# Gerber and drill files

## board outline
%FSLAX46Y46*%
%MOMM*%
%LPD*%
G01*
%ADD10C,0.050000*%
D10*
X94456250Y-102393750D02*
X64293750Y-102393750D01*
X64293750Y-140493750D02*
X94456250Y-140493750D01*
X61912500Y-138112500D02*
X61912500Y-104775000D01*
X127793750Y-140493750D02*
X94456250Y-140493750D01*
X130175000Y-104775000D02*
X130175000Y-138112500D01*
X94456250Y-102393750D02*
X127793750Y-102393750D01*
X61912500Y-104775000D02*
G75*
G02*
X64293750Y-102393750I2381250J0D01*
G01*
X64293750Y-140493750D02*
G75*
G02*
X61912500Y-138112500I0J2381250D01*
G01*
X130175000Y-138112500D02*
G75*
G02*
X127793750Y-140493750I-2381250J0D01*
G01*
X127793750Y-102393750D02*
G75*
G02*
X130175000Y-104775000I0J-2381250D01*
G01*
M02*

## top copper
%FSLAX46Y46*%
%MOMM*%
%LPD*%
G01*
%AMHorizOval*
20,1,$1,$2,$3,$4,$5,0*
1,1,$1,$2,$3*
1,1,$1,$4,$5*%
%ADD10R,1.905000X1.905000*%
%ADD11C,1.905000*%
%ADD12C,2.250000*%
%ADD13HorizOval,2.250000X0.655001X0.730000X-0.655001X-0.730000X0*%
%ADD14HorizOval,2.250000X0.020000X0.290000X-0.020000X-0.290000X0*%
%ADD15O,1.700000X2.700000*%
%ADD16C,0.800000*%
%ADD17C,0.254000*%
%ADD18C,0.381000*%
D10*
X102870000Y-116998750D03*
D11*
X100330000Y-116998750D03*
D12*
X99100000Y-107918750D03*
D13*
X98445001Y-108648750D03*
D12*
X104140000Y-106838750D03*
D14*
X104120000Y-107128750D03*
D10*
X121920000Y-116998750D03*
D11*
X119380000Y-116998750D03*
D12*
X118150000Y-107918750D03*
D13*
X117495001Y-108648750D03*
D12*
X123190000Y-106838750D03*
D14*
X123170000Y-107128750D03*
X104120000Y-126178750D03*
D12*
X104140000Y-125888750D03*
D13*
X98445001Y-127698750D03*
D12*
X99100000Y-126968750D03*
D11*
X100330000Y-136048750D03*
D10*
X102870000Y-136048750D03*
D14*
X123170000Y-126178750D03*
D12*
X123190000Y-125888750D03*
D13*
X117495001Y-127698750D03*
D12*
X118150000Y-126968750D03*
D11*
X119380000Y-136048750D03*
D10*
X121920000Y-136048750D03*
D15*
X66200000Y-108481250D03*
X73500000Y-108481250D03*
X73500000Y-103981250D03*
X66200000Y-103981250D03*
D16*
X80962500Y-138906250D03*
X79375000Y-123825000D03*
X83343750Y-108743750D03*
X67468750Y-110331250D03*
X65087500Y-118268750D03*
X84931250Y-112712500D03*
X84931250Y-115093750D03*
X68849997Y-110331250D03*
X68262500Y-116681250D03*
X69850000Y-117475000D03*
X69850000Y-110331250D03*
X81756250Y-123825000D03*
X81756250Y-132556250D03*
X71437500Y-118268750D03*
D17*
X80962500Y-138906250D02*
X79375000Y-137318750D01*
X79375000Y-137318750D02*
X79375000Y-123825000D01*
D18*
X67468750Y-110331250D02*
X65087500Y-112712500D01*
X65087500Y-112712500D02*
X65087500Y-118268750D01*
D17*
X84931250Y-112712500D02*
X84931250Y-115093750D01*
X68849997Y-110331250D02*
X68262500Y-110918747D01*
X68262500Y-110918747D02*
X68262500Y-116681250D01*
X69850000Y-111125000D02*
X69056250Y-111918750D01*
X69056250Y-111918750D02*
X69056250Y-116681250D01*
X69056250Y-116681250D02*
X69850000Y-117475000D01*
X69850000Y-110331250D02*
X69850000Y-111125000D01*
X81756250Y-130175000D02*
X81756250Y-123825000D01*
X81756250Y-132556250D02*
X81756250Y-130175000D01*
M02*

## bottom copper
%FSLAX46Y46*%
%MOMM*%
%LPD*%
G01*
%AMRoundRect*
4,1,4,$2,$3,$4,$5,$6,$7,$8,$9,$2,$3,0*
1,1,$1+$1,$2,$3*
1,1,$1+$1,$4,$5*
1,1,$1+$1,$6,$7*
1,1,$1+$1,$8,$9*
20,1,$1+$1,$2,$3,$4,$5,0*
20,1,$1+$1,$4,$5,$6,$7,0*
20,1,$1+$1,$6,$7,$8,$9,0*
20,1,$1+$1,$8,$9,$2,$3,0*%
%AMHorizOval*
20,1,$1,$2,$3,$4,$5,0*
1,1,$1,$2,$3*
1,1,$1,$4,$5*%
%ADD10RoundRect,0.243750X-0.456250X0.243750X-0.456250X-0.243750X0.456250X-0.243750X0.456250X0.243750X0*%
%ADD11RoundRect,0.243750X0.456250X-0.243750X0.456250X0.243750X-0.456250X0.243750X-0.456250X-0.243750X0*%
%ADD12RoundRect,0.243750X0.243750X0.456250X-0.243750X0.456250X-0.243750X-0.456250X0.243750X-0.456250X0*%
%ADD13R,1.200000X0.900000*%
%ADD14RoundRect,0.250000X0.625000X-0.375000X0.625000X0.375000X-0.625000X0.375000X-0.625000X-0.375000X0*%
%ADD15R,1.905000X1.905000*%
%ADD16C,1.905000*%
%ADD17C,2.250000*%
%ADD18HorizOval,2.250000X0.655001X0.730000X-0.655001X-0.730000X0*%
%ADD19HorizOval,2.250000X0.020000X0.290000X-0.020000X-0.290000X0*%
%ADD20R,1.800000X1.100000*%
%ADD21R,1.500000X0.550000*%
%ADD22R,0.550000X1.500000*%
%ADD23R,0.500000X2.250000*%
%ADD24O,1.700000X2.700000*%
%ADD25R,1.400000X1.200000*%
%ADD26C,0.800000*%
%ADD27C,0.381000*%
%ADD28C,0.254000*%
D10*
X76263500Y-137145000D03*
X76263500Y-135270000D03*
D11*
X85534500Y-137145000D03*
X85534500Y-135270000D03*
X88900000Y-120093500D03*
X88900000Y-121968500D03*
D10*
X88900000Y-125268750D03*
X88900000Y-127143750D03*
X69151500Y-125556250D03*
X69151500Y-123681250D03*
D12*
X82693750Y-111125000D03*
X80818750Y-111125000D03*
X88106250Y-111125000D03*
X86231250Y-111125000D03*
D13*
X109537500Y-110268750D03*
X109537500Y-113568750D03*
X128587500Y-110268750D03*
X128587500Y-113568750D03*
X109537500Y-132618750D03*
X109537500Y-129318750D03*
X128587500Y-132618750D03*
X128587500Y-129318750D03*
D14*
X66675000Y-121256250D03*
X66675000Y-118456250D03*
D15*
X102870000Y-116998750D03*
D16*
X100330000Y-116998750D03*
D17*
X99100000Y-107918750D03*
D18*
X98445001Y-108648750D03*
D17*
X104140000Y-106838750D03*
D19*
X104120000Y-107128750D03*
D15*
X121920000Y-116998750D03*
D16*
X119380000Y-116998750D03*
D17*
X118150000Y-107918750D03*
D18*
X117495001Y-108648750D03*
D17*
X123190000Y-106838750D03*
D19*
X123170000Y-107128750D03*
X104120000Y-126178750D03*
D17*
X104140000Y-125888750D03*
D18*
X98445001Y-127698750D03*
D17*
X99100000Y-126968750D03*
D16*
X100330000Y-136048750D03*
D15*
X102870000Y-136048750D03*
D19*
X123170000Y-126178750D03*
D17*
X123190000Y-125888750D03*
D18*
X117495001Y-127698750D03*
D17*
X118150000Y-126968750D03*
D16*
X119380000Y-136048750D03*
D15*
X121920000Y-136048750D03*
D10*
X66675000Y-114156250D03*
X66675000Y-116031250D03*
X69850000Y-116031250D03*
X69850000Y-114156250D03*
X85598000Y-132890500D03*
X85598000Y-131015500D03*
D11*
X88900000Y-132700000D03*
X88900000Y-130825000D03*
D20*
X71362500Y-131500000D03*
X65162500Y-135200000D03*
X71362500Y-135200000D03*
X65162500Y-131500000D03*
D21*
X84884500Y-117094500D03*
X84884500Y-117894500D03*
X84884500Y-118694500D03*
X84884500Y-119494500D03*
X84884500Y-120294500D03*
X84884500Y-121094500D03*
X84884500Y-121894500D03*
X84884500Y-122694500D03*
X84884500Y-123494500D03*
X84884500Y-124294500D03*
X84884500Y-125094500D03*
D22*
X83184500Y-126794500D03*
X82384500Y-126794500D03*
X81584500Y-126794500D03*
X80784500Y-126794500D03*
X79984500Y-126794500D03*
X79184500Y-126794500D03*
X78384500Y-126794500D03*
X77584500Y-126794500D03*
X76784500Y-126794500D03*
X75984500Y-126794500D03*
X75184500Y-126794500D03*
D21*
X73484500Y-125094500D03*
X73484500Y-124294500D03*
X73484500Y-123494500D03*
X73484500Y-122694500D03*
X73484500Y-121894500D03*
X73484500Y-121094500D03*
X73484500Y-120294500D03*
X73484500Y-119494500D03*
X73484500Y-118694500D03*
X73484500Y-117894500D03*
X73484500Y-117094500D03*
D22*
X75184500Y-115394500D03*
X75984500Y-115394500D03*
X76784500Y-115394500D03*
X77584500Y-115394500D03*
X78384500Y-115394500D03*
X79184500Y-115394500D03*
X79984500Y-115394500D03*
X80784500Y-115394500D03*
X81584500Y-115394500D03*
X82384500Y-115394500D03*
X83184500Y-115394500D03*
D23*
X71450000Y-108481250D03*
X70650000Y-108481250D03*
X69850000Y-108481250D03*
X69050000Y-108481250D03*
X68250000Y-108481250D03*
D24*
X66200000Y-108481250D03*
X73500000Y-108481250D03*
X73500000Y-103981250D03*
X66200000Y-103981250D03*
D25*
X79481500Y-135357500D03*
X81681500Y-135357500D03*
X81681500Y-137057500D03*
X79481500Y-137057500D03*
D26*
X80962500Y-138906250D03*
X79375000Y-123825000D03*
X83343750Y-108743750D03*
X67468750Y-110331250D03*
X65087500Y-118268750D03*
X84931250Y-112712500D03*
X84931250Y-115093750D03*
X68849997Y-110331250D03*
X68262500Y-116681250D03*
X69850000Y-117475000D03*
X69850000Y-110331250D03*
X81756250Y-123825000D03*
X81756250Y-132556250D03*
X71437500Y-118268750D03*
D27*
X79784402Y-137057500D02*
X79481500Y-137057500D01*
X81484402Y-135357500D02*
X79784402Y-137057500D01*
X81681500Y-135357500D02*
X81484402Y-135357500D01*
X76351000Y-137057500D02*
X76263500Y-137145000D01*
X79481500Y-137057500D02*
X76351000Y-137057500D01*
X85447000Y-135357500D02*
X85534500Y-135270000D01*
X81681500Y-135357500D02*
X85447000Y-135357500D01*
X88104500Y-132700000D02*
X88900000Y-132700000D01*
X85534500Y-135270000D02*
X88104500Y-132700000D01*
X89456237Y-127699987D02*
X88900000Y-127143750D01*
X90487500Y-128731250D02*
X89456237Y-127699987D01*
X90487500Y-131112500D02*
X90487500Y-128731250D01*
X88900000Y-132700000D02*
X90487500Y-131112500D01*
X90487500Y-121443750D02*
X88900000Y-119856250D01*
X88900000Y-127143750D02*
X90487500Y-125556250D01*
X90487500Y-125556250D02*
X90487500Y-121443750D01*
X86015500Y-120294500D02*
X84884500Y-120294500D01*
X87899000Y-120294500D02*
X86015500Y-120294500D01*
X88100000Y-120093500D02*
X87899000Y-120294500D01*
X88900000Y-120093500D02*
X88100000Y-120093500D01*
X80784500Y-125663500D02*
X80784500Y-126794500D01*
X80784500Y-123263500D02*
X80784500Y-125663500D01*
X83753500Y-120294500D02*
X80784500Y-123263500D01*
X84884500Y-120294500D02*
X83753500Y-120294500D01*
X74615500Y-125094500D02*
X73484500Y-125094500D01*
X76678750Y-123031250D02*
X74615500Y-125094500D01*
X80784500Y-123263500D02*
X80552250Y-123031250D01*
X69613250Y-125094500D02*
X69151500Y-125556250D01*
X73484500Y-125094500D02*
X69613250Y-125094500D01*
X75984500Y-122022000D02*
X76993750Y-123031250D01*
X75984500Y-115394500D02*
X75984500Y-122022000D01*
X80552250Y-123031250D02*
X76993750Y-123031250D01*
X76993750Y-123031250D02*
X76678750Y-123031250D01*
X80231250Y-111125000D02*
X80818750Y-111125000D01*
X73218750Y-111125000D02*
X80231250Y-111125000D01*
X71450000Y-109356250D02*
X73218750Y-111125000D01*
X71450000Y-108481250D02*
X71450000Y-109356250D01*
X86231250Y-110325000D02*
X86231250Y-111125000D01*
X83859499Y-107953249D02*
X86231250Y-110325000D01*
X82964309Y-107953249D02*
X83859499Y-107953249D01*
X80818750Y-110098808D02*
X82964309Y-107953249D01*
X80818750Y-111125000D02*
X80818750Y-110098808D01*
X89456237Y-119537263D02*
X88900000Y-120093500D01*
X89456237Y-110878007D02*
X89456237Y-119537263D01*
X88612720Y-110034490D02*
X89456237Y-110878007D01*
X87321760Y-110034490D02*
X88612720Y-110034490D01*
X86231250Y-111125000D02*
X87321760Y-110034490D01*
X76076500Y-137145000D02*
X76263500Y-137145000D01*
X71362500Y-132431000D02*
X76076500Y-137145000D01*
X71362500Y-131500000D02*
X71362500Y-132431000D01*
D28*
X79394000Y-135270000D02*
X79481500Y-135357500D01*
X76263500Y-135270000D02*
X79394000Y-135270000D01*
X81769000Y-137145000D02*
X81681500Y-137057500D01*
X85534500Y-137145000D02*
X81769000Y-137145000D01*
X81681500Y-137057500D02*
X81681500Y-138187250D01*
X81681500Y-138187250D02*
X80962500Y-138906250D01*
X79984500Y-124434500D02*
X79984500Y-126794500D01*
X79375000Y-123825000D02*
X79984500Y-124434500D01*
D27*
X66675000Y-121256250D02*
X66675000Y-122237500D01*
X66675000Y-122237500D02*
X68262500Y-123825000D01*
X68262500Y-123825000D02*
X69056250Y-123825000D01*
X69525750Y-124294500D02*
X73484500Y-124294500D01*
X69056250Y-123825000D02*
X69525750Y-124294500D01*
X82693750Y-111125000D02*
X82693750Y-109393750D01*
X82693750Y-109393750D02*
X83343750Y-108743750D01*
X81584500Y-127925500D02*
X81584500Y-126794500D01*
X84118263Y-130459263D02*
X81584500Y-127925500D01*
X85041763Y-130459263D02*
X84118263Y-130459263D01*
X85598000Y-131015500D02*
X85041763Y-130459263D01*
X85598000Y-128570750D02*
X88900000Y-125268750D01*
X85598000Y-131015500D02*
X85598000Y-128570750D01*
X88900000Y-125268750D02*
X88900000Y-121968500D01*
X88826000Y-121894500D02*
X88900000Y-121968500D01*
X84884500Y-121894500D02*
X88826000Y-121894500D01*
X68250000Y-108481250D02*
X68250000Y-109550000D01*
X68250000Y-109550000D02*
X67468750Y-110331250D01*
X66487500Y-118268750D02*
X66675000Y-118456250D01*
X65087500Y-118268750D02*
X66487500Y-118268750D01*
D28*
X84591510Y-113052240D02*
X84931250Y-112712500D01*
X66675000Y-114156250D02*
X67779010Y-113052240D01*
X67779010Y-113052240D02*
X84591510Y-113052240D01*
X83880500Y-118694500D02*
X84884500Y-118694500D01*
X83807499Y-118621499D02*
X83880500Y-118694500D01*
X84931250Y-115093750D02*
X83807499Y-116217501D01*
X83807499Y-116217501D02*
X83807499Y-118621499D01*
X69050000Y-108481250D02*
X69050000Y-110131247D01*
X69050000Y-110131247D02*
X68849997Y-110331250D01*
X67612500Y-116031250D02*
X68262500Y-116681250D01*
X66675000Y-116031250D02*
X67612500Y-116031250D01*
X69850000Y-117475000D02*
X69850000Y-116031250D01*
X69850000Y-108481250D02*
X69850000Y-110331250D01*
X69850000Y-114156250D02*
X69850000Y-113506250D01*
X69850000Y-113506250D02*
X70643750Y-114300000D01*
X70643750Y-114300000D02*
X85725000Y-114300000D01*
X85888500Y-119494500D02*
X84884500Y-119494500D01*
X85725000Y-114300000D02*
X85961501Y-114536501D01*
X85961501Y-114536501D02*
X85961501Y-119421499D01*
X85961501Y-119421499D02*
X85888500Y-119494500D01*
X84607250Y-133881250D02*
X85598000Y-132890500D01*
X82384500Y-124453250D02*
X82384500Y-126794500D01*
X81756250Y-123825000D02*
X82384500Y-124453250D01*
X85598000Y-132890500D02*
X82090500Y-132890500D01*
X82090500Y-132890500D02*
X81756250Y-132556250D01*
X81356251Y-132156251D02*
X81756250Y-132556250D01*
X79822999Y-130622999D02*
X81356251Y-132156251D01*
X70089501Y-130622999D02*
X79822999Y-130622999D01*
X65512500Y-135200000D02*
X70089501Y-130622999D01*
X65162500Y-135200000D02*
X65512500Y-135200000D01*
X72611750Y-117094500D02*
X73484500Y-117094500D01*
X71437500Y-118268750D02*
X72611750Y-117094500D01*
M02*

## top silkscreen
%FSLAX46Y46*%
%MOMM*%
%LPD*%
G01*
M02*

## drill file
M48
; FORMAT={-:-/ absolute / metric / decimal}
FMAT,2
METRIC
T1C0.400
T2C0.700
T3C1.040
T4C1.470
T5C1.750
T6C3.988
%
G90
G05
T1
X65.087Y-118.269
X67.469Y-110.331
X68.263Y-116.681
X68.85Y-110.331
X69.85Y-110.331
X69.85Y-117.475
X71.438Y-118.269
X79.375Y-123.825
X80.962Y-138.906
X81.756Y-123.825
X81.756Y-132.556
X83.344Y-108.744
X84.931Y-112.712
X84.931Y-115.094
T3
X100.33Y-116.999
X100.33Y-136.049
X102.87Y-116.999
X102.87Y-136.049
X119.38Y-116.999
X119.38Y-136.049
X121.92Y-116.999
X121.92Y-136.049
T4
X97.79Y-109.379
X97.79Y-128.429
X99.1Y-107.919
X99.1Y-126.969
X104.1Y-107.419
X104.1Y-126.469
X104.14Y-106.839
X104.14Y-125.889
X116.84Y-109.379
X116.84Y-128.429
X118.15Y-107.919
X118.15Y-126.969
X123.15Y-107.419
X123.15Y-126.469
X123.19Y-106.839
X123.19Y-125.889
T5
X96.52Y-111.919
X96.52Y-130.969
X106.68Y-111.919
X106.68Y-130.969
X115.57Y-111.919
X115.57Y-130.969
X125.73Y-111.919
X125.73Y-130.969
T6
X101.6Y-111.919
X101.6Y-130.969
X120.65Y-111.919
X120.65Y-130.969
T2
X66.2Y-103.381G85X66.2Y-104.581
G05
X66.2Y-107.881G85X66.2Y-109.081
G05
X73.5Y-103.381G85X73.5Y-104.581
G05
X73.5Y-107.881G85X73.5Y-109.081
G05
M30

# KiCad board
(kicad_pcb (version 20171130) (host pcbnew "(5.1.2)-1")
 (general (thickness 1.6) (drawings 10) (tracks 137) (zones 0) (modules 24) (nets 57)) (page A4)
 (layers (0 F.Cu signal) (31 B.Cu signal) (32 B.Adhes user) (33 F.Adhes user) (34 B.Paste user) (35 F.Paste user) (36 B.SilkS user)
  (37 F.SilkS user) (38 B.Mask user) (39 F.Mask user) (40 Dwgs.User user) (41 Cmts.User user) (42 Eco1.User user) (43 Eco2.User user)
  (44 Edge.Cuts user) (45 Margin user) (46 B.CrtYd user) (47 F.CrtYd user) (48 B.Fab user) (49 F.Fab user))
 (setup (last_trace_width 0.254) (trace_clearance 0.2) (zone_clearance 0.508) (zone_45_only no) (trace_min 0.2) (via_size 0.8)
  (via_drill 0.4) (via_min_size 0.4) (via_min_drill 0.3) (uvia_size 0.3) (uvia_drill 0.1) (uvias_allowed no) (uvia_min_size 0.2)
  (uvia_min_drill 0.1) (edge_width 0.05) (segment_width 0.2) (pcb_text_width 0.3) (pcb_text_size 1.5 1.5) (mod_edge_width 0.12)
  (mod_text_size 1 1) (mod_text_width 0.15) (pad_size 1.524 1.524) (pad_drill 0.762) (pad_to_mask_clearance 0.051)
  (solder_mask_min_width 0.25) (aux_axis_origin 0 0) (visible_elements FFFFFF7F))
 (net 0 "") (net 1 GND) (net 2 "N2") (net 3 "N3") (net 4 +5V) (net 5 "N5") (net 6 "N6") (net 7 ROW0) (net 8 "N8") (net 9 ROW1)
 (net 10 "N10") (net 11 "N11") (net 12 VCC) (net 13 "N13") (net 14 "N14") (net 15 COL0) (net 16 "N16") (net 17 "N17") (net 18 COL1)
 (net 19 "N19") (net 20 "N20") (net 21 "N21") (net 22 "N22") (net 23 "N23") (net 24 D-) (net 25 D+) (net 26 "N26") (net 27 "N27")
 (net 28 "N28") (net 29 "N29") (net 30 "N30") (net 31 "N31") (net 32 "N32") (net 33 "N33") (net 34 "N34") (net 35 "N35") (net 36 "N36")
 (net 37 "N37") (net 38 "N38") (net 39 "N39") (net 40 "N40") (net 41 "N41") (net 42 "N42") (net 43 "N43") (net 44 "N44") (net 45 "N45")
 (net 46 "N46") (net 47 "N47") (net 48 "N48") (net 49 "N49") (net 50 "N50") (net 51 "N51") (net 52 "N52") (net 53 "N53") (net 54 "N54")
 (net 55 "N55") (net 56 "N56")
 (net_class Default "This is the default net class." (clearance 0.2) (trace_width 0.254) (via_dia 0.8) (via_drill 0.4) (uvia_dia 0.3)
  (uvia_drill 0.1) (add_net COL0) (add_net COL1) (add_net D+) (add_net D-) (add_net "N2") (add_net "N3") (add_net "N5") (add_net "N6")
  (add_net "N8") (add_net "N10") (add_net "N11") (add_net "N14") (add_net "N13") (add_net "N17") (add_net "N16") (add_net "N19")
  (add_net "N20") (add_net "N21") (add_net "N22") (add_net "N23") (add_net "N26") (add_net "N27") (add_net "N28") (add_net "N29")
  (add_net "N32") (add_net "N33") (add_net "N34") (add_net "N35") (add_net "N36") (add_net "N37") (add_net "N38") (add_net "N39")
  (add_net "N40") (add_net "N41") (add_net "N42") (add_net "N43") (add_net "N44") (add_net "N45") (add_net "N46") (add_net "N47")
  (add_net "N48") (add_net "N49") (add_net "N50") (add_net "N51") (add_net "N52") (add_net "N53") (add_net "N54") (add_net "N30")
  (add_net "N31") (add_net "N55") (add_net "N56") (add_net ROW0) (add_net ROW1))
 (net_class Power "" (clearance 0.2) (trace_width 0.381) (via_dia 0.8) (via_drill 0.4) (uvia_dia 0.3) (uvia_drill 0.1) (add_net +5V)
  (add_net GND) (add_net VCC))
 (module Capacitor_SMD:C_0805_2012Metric (layer B.Cu) (at 76.2635 136.2075 270)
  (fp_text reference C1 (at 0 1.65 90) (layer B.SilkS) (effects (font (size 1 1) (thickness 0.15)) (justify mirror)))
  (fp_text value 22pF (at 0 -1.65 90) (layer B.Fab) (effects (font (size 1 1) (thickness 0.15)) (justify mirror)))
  (pad 2 smd roundrect (at 0.9375 0 270) (size 0.975 1.4) (layers B.Cu B.Paste B.Mask) (roundrect_rratio 0.25) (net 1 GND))
  (pad 1 smd roundrect (at -0.9375 0 270) (size 0.975 1.4) (layers B.Cu B.Paste B.Mask) (roundrect_rratio 0.25) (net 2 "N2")))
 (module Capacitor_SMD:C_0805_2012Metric (layer B.Cu) (at 85.5345 136.2075 90)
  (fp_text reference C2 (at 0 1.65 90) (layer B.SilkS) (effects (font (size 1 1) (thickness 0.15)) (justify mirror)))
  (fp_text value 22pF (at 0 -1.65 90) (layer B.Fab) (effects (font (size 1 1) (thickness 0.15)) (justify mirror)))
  (pad 1 smd roundrect (at -0.9375 0 90) (size 0.975 1.4) (layers B.Cu B.Paste B.Mask) (roundrect_rratio 0.25) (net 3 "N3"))
  (pad 2 smd roundrect (at 0.9375 0 90) (size 0.975 1.4) (layers B.Cu B.Paste B.Mask) (roundrect_rratio 0.25) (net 1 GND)))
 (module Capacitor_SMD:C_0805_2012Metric (layer B.Cu) (at 88.9 121.031 90)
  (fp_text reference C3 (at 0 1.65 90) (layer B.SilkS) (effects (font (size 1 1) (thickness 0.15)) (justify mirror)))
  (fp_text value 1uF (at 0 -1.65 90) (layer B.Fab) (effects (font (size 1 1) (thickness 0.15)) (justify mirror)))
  (pad 2 smd roundrect (at 0.9375 0 90) (size 0.975 1.4) (layers B.Cu B.Paste B.Mask) (roundrect_rratio 0.25) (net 1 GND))
  (pad 1 smd roundrect (at -0.9375 0 90) (size 0.975 1.4) (layers B.Cu B.Paste B.Mask) (roundrect_rratio 0.25) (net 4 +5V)))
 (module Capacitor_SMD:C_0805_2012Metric (layer B.Cu) (at 88.9 126.20625 270)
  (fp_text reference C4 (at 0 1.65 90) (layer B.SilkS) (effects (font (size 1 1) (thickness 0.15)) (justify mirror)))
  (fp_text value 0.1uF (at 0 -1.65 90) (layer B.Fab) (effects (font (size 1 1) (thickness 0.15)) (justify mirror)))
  (pad 1 smd roundrect (at -0.9375 0 270) (size 0.975 1.4) (layers B.Cu B.Paste B.Mask) (roundrect_rratio 0.25) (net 4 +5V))
  (pad 2 smd roundrect (at 0.9375 0 270) (size 0.975 1.4) (layers B.Cu B.Paste B.Mask) (roundrect_rratio 0.25) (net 1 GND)))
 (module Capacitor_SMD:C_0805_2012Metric (layer B.Cu) (at 69.1515 124.61875 270)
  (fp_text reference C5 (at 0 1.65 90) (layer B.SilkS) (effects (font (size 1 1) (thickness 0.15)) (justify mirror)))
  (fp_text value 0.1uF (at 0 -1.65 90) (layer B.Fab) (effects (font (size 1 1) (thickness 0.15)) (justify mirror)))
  (pad 2 smd roundrect (at 0.9375 0 270) (size 0.975 1.4) (layers B.Cu B.Paste B.Mask) (roundrect_rratio 0.25) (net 1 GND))
  (pad 1 smd roundrect (at -0.9375 0 270) (size 0.975 1.4) (layers B.Cu B.Paste B.Mask) (roundrect_rratio 0.25) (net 4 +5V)))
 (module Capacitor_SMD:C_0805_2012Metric (layer B.Cu) (at 81.75625 111.125 180)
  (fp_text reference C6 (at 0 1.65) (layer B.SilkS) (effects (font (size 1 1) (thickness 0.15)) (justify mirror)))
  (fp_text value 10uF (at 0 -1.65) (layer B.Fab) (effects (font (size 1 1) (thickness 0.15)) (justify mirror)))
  (pad 1 smd roundrect (at -0.9375 0 180) (size 0.975 1.4) (layers B.Cu B.Paste B.Mask) (roundrect_rratio 0.25) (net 4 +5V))
  (pad 2 smd roundrect (at 0.9375 0 180) (size 0.975 1.4) (layers B.Cu B.Paste B.Mask) (roundrect_rratio 0.25) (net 1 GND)))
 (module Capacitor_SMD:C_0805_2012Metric (layer B.Cu) (at 87.16875 111.125 180)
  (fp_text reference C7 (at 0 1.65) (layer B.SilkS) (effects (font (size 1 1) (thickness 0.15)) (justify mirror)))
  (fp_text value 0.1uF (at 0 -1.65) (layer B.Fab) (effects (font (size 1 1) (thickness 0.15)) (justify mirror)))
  (pad 1 smd roundrect (at -0.9375 0 180) (size 0.975 1.4) (layers B.Cu B.Paste B.Mask) (roundrect_rratio 0.25) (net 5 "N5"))
  (pad 2 smd roundrect (at 0.9375 0 180) (size 0.975 1.4) (layers B.Cu B.Paste B.Mask) (roundrect_rratio 0.25) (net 1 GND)))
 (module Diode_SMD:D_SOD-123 (layer B.Cu) (at 109.5375 111.91875 90)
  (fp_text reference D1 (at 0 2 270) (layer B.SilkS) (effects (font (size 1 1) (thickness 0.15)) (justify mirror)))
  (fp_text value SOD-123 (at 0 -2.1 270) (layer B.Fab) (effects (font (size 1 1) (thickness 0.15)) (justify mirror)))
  (pad 2 smd rect (at 1.65 0 90) (size 0.9 1.2) (layers B.Cu B.Paste B.Mask) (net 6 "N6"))
  (pad 1 smd rect (at -1.65 0 90) (size 0.9 1.2) (layers B.Cu B.Paste B.Mask) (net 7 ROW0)))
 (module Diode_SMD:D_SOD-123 (layer B.Cu) (at 128.5875 111.91875 90)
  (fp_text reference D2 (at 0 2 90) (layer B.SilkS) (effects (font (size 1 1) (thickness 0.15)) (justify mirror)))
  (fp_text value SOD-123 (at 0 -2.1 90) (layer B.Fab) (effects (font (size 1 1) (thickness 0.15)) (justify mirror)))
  (pad 2 smd rect (at 1.65 0 90) (size 0.9 1.2) (layers B.Cu B.Paste B.Mask) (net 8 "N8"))
  (pad 1 smd rect (at -1.65 0 90) (size 0.9 1.2) (layers B.Cu B.Paste B.Mask) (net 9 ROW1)))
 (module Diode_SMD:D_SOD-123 (layer B.Cu) (at 109.5375 130.96875 90)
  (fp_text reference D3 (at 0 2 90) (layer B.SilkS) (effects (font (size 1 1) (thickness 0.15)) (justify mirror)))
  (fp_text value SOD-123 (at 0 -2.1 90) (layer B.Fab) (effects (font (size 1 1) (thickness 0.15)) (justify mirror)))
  (pad 1 smd rect (at -1.65 0 90) (size 0.9 1.2) (layers B.Cu B.Paste B.Mask) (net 7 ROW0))
  (pad 2 smd rect (at 1.65 0 90) (size 0.9 1.2) (layers B.Cu B.Paste B.Mask) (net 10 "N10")))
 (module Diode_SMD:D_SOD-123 (layer B.Cu) (at 128.5875 130.96875 90)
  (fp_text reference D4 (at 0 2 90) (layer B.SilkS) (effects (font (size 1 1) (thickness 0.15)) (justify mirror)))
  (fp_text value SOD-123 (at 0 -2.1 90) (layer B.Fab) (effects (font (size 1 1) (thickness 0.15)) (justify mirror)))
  (pad 1 smd rect (at -1.65 0 90) (size 0.9 1.2) (layers B.Cu B.Paste B.Mask) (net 9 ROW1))
  (pad 2 smd rect (at 1.65 0 90) (size 0.9 1.2) (layers B.Cu B.Paste B.Mask) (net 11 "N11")))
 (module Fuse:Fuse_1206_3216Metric (layer B.Cu) (at 66.675 119.85625 90)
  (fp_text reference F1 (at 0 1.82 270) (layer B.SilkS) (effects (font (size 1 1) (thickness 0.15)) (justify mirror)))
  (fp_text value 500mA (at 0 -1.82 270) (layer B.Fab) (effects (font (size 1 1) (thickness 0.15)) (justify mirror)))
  (pad 1 smd roundrect (at -1.4 0 90) (size 1.25 1.75) (layers B.Cu B.Paste B.Mask) (roundrect_rratio 0.2) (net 4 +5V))
  (pad 2 smd roundrect (at 1.4 0 90) (size 1.25 1.75) (layers B.Cu B.Paste B.Mask) (roundrect_rratio 0.2) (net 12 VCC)))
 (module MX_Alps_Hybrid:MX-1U (layer F.Cu) (at 101.6 111.91875)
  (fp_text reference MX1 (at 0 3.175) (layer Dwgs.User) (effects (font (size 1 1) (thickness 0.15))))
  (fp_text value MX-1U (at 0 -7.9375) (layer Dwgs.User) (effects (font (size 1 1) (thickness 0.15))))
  (pad "" np_thru_hole circle (at 5.08 0 48.0996) (size 1.75 1.75) (drill 1.75) (layers *.Cu *.Mask))
  (pad "" np_thru_hole circle (at -5.08 0 48.0996) (size 1.75 1.75) (drill 1.75) (layers *.Cu *.Mask))
  (pad 4 thru_hole rect (at 1.27 5.08) (size 1.905 1.905) (drill 1.04) (layers *.Cu B.Mask) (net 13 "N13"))
  (pad 3 thru_hole circle (at -1.27 5.08) (size 1.905 1.905) (drill 1.04) (layers *.Cu B.Mask) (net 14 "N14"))
  (pad 1 thru_hole circle (at -2.5 -4) (size 2.25 2.25) (drill 1.47) (layers *.Cu B.Mask) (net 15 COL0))
  (pad "" np_thru_hole circle (at 0 0) (size 3.9878 3.9878) (drill 3.9878) (layers *.Cu *.Mask))
  (pad 1 thru_hole oval (at -3.81 -2.54 48.0996) (size 4.211556 2.25) (drill 1.47 (offset 0.980778 0)) (layers *.Cu B.Mask) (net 15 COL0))
  (pad 2 thru_hole circle (at 2.54 -5.08) (size 2.25 2.25) (drill 1.47) (layers *.Cu B.Mask) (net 6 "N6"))
  (pad 2 thru_hole oval (at 2.5 -4.5 86.0548) (size 2.831378 2.25) (drill 1.47 (offset 0.290689 0)) (layers *.Cu B.Mask) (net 6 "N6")))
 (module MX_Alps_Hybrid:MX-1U (layer F.Cu) (at 120.65 111.91875)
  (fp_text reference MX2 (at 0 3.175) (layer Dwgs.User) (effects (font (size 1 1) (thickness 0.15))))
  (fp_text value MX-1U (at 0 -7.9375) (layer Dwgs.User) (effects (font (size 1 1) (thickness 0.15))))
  (pad "" np_thru_hole circle (at 5.08 0 48.0996) (size 1.75 1.75) (drill 1.75) (layers *.Cu *.Mask))
  (pad "" np_thru_hole circle (at -5.08 0 48.0996) (size 1.75 1.75) (drill 1.75) (layers *.Cu *.Mask))
  (pad 4 thru_hole rect (at 1.27 5.08) (size 1.905 1.905) (drill 1.04) (layers *.Cu B.Mask) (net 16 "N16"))
  (pad 3 thru_hole circle (at -1.27 5.08) (size 1.905 1.905) (drill 1.04) (layers *.Cu B.Mask) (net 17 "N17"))
  (pad 1 thru_hole circle (at -2.5 -4) (size 2.25 2.25) (drill 1.47) (layers *.Cu B.Mask) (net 15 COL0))
  (pad "" np_thru_hole circle (at 0 0) (size 3.9878 3.9878) (drill 3.9878) (layers *.Cu *.Mask))
  (pad 1 thru_hole oval (at -3.81 -2.54 48.0996) (size 4.211556 2.25) (drill 1.47 (offset 0.980778 0)) (layers *.Cu B.Mask) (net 15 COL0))
  (pad 2 thru_hole circle (at 2.54 -5.08) (size 2.25 2.25) (drill 1.47) (layers *.Cu B.Mask) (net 8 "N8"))
  (pad 2 thru_hole oval (at 2.5 -4.5 86.0548) (size 2.831378 2.25) (drill 1.47 (offset 0.290689 0)) (layers *.Cu B.Mask) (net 8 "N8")))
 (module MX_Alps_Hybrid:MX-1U (layer F.Cu) (at 101.6 130.96875)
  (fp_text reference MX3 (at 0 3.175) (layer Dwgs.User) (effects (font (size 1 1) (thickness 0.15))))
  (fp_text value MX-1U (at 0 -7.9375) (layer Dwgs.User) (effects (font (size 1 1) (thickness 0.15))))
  (pad 2 thru_hole oval (at 2.5 -4.5 86.0548) (size 2.831378 2.25) (drill 1.47 (offset 0.290689 0)) (layers *.Cu B.Mask) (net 10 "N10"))
  (pad 2 thru_hole circle (at 2.54 -5.08) (size 2.25 2.25) (drill 1.47) (layers *.Cu B.Mask) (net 10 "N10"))
  (pad 1 thru_hole oval (at -3.81 -2.54 48.0996) (size 4.211556 2.25) (drill 1.47 (offset 0.980778 0)) (layers *.Cu B.Mask) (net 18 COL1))
  (pad "" np_thru_hole circle (at 0 0) (size 3.9878 3.9878) (drill 3.9878) (layers *.Cu *.Mask))
  (pad 1 thru_hole circle (at -2.5 -4) (size 2.25 2.25) (drill 1.47) (layers *.Cu B.Mask) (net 18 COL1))
  (pad 3 thru_hole circle (at -1.27 5.08) (size 1.905 1.905) (drill 1.04) (layers *.Cu B.Mask) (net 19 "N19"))
  (pad 4 thru_hole rect (at 1.27 5.08) (size 1.905 1.905) (drill 1.04) (layers *.Cu B.Mask) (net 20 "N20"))
  (pad "" np_thru_hole circle (at -5.08 0 48.0996) (size 1.75 1.75) (drill 1.75) (layers *.Cu *.Mask))
  (pad "" np_thru_hole circle (at 5.08 0 48.0996) (size 1.75 1.75) (drill 1.75) (layers *.Cu *.Mask)))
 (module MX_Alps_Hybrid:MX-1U (layer F.Cu) (at 120.65 130.96875)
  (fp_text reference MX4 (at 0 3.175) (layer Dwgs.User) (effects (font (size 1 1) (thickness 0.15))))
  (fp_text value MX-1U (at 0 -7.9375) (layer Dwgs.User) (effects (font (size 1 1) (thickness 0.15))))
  (pad 2 thru_hole oval (at 2.5 -4.5 86.0548) (size 2.831378 2.25) (drill 1.47 (offset 0.290689 0)) (layers *.Cu B.Mask) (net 11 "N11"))
  (pad 2 thru_hole circle (at 2.54 -5.08) (size 2.25 2.25) (drill 1.47) (layers *.Cu B.Mask) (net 11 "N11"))
  (pad 1 thru_hole oval (at -3.81 -2.54 48.0996) (size 4.211556 2.25) (drill 1.47 (offset 0.980778 0)) (layers *.Cu B.Mask) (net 18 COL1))
  (pad "" np_thru_hole circle (at 0 0) (size 3.9878 3.9878) (drill 3.9878) (layers *.Cu *.Mask))
  (pad 1 thru_hole circle (at -2.5 -4) (size 2.25 2.25) (drill 1.47) (layers *.Cu B.Mask) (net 18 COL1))
  (pad 3 thru_hole circle (at -1.27 5.08) (size 1.905 1.905) (drill 1.04) (layers *.Cu B.Mask) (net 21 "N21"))
  (pad 4 thru_hole rect (at 1.27 5.08) (size 1.905 1.905) (drill 1.04) (layers *.Cu B.Mask) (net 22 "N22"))
  (pad "" np_thru_hole circle (at -5.08 0 48.0996) (size 1.75 1.75) (drill 1.75) (layers *.Cu *.Mask))
  (pad "" np_thru_hole circle (at 5.08 0 48.0996) (size 1.75 1.75) (drill 1.75) (layers *.Cu *.Mask)))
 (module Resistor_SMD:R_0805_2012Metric (layer B.Cu) (at 66.675 115.09375 270)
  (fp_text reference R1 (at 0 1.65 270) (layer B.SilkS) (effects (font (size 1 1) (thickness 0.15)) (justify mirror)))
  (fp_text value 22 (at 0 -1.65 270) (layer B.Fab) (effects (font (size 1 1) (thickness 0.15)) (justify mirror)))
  (pad 1 smd roundrect (at -0.9375 0 270) (size 0.975 1.4) (layers B.Cu B.Paste B.Mask) (roundrect_rratio 0.25) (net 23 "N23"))
  (pad 2 smd roundrect (at 0.9375 0 270) (size 0.975 1.4) (layers B.Cu B.Paste B.Mask) (roundrect_rratio 0.25) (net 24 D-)))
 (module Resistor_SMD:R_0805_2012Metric (layer B.Cu) (at 69.85 115.09375 270)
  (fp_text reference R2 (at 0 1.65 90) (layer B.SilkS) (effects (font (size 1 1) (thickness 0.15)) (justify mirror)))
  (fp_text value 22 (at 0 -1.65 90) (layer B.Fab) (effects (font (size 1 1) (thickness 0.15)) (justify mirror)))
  (pad 2 smd roundrect (at 0.9375 0 270) (size 0.975 1.4) (layers B.Cu B.Paste B.Mask) (roundrect_rratio 0.25) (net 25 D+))
  (pad 1 smd roundrect (at -0.9375 0 270) (size 0.975 1.4) (layers B.Cu B.Paste B.Mask) (roundrect_rratio 0.25) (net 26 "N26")))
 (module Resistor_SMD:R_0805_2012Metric (layer B.Cu) (at 85.598 131.953 270)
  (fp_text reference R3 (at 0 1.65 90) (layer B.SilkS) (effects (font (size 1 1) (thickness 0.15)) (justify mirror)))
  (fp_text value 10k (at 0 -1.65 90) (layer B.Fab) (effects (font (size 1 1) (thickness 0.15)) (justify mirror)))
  (pad 2 smd roundrect (at 0.9375 0 270) (size 0.975 1.4) (layers B.Cu B.Paste B.Mask) (roundrect_rratio 0.25) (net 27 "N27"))
  (pad 1 smd roundrect (at -0.9375 0 270) (size 0.975 1.4) (layers B.Cu B.Paste B.Mask) (roundrect_rratio 0.25) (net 4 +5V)))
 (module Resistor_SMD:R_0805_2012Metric (layer B.Cu) (at 88.9 131.7625 90)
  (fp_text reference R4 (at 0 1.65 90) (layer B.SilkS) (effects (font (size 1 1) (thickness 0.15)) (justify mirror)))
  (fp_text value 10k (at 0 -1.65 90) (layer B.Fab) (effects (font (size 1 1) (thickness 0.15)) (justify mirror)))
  (pad 1 smd roundrect (at -0.9375 0 90) (size 0.975 1.4) (layers B.Cu B.Paste B.Mask) (roundrect_rratio 0.25) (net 1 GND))
  (pad 2 smd roundrect (at 0.9375 0 90) (size 0.975 1.4) (layers B.Cu B.Paste B.Mask) (roundrect_rratio 0.25) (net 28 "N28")))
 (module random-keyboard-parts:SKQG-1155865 (layer B.Cu) (at 68.2625 133.35)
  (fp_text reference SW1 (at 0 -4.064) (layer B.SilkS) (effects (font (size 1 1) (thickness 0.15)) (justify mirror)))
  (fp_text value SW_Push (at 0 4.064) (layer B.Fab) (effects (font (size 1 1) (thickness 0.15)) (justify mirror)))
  (pad 1 smd rect (at 3.1 -1.85) (size 1.8 1.1) (layers B.Cu B.Paste B.Mask) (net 1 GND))
  (pad 2 smd rect (at -3.1 1.85) (size 1.8 1.1) (layers B.Cu B.Paste B.Mask) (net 27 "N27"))
  (pad 3 smd rect (at 3.1 1.85) (size 1.8 1.1) (layers B.Cu B.Paste B.Mask))
  (pad 4 smd rect (at -3.1 -1.85) (size 1.8 1.1) (layers B.Cu B.Paste B.Mask)))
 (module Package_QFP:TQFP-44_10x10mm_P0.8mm (layer B.Cu) (at 79.1845 121.0945 180)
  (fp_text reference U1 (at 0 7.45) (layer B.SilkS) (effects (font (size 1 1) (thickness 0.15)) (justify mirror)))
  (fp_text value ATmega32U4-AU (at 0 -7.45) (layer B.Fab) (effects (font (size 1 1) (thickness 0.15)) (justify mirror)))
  (pad 1 smd rect (at -5.7 4 180) (size 1.5 0.55) (layers B.Cu B.Paste B.Mask) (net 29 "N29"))
  (pad 2 smd rect (at -5.7 3.2 180) (size 1.5 0.55) (layers B.Cu B.Paste B.Mask) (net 4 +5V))
  (pad 3 smd rect (at -5.7 2.4 180) (size 1.5 0.55) (layers B.Cu B.Paste B.Mask) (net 23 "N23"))
  (pad 4 smd rect (at -5.7 1.6 180) (size 1.5 0.55) (layers B.Cu B.Paste B.Mask) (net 26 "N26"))
  (pad 5 smd rect (at -5.7 0.8 180) (size 1.5 0.55) (layers B.Cu B.Paste B.Mask) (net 1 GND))
  (pad 6 smd rect (at -5.7 0 180) (size 1.5 0.55) (layers B.Cu B.Paste B.Mask) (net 5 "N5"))
  (pad 7 smd rect (at -5.7 -0.8 180) (size 1.5 0.55) (layers B.Cu B.Paste B.Mask) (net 4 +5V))
  (pad 8 smd rect (at -5.7 -1.6 180) (size 1.5 0.55) (layers B.Cu B.Paste B.Mask) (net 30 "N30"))
  (pad 9 smd rect (at -5.7 -2.4 180) (size 1.5 0.55) (layers B.Cu B.Paste B.Mask) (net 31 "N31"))
  (pad 10 smd rect (at -5.7 -3.2 180) (size 1.5 0.55) (layers B.Cu B.Paste B.Mask) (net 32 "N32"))
  (pad 11 smd rect (at -5.7 -4 180) (size 1.5 0.55) (layers B.Cu B.Paste B.Mask) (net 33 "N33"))
  (pad 12 smd rect (at -4 -5.7 90) (size 1.5 0.55) (layers B.Cu B.Paste B.Mask) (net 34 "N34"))
  (pad 13 smd rect (at -3.2 -5.7 90) (size 1.5 0.55) (layers B.Cu B.Paste B.Mask) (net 27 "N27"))
  (pad 14 smd rect (at -2.4 -5.7 90) (size 1.5 0.55) (layers B.Cu B.Paste B.Mask) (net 4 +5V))
  (pad 15 smd rect (at -1.6 -5.7 90) (size 1.5 0.55) (layers B.Cu B.Paste B.Mask) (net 1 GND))
  (pad 16 smd rect (at -0.8 -5.7 90) (size 1.5 0.55) (layers B.Cu B.Paste B.Mask) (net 3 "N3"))
  (pad 17 smd rect (at 0 -5.7 90) (size 1.5 0.55) (layers B.Cu B.Paste B.Mask) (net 2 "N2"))
  (pad 18 smd rect (at 0.8 -5.7 90) (size 1.5 0.55) (layers B.Cu B.Paste B.Mask) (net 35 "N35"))
  (pad 19 smd rect (at 1.6 -5.7 90) (size 1.5 0.55) (layers B.Cu B.Paste B.Mask) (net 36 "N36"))
  (pad 20 smd rect (at 2.4 -5.7 90) (size 1.5 0.55) (layers B.Cu B.Paste B.Mask) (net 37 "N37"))
  (pad 21 smd rect (at 3.2 -5.7 90) (size 1.5 0.55) (layers B.Cu B.Paste B.Mask) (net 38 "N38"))
  (pad 22 smd rect (at 4 -5.7 90) (size 1.5 0.55) (layers B.Cu B.Paste B.Mask) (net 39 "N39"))
  (pad 23 smd rect (at 5.7 -4 180) (size 1.5 0.55) (layers B.Cu B.Paste B.Mask) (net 1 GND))
  (pad 24 smd rect (at 5.7 -3.2 180) (size 1.5 0.55) (layers B.Cu B.Paste B.Mask) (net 4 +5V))
  (pad 25 smd rect (at 5.7 -2.4 180) (size 1.5 0.55) (layers B.Cu B.Paste B.Mask) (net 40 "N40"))
  (pad 26 smd rect (at 5.7 -1.6 180) (size 1.5 0.55) (layers B.Cu B.Paste B.Mask) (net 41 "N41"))
  (pad 27 smd rect (at 5.7 -0.8 180) (size 1.5 0.55) (layers B.Cu B.Paste B.Mask) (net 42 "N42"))
  (pad 28 smd rect (at 5.7 0 180) (size 1.5 0.55) (layers B.Cu B.Paste B.Mask) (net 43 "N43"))
  (pad 29 smd rect (at 5.7 0.8 180) (size 1.5 0.55) (layers B.Cu B.Paste B.Mask) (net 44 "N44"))
  (pad 30 smd rect (at 5.7 1.6 180) (size 1.5 0.55) (layers B.Cu B.Paste B.Mask) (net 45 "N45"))
  (pad 31 smd rect (at 5.7 2.4 180) (size 1.5 0.55) (layers B.Cu B.Paste B.Mask) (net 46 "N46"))
  (pad 32 smd rect (at 5.7 3.2 180) (size 1.5 0.55) (layers B.Cu B.Paste B.Mask) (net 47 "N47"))
  (pad 33 smd rect (at 5.7 4 180) (size 1.5 0.55) (layers B.Cu B.Paste B.Mask) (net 28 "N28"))
  (pad 34 smd rect (at 4 5.7 90) (size 1.5 0.55) (layers B.Cu B.Paste B.Mask) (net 4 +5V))
  (pad 35 smd rect (at 3.2 5.7 90) (size 1.5 0.55) (layers B.Cu B.Paste B.Mask) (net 1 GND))
  (pad 36 smd rect (at 2.4 5.7 90) (size 1.5 0.55) (layers B.Cu B.Paste B.Mask) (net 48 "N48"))
  (pad 37 smd rect (at 1.6 5.7 90) (size 1.5 0.55) (layers B.Cu B.Paste B.Mask) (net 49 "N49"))
  (pad 38 smd rect (at 0.8 5.7 90) (size 1.5 0.55) (layers B.Cu B.Paste B.Mask) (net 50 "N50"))
  (pad 39 smd rect (at 0 5.7 90) (size 1.5 0.55) (layers B.Cu B.Paste B.Mask) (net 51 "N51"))
  (pad 40 smd rect (at -0.8 5.7 90) (size 1.5 0.55) (layers B.Cu B.Paste B.Mask) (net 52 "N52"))
  (pad 41 smd rect (at -1.6 5.7 90) (size 1.5 0.55) (layers B.Cu B.Paste B.Mask) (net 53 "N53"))
  (pad 42 smd rect (at -2.4 5.7 90) (size 1.5 0.55) (layers B.Cu B.Paste B.Mask) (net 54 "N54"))
  (pad 43 smd rect (at -3.2 5.7 90) (size 1.5 0.55) (layers B.Cu B.Paste B.Mask) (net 1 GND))
  (pad 44 smd rect (at -4 5.7 90) (size 1.5 0.55) (layers B.Cu B.Paste B.Mask) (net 4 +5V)))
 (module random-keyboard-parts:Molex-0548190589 (layer B.Cu) (at 69.85 103.98125 270)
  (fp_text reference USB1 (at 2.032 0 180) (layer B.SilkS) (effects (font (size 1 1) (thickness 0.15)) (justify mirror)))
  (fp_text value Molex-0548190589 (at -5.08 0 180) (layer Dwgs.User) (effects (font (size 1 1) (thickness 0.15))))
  (pad 1 smd rect (at 4.5 -1.6 270) (size 2.25 0.5) (layers B.Cu B.Paste B.Mask) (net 1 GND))
  (pad 2 smd rect (at 4.5 -0.8 270) (size 2.25 0.5) (layers B.Cu B.Paste B.Mask) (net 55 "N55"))
  (pad 3 smd rect (at 4.5 0 270) (size 2.25 0.5) (layers B.Cu B.Paste B.Mask) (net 25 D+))
  (pad 4 smd rect (at 4.5 0.8 270) (size 2.25 0.5) (layers B.Cu B.Paste B.Mask) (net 24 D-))
  (pad 5 smd rect (at 4.5 1.6 270) (size 2.25 0.5) (layers B.Cu B.Paste B.Mask) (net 12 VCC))
  (pad 6 thru_hole oval (at 4.5 3.65 270) (size 2.7 1.7) (drill oval 1.9 0.7) (layers *.Cu *.Mask) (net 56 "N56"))
  (pad 6 thru_hole oval (at 4.5 -3.65 270) (size 2.7 1.7) (drill oval 1.9 0.7) (layers *.Cu *.Mask) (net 56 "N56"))
  (pad 6 thru_hole oval (at 0 -3.65 270) (size 2.7 1.7) (drill oval 1.9 0.7) (layers *.Cu *.Mask) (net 56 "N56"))
  (pad 6 thru_hole oval (at 0 3.65 270) (size 2.7 1.7) (drill oval 1.9 0.7) (layers *.Cu *.Mask) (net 56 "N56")))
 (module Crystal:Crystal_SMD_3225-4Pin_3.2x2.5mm (layer B.Cu) (at 80.5815 136.2075)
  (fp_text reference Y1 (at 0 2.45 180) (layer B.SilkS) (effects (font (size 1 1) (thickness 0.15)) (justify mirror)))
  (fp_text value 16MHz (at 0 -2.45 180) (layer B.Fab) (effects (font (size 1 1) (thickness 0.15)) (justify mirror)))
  (pad 1 smd rect (at -1.1 -0.85) (size 1.4 1.2) (layers B.Cu B.Paste B.Mask) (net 2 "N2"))
  (pad 2 smd rect (at 1.1 -0.85) (size 1.4 1.2) (layers B.Cu B.Paste B.Mask) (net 1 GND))
  (pad 3 smd rect (at 1.1 0.85) (size 1.4 1.2) (layers B.Cu B.Paste B.Mask) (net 3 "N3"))
  (pad 4 smd rect (at -1.1 0.85) (size 1.4 1.2) (layers B.Cu B.Paste B.Mask) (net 1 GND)))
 (gr_line (start 94.45625 102.39375) (end 64.29375 102.39375) (layer Edge.Cuts) (width 0.05))
 (gr_line (start 64.29375 140.49375) (end 94.45625 140.49375) (layer Edge.Cuts) (width 0.05))
 (gr_line (start 61.9125 138.1125) (end 61.9125 104.775) (layer Edge.Cuts) (width 0.05))
 (gr_line (start 127.79375 140.49375) (end 94.45625 140.49375) (layer Edge.Cuts) (width 0.05))
 (gr_line (start 130.175 104.775) (end 130.175 138.1125) (layer Edge.Cuts) (width 0.05))
 (gr_line (start 94.45625 102.39375) (end 127.79375 102.39375) (layer Edge.Cuts) (width 0.05))
 (gr_arc (start 64.29375 104.775) (end 64.29375 102.39375) (angle -90) (layer Edge.Cuts) (width 0.05))
 (gr_arc (start 64.29375 138.1125) (end 61.9125 138.1125) (angle -90) (layer Edge.Cuts) (width 0.05))
 (gr_arc (start 127.79375 138.1125) (end 127.79375 140.49375) (angle -90) (layer Edge.Cuts) (width 0.05))
 (gr_arc (start 127.79375 104.775) (end 130.175 104.775) (angle -90) (layer Edge.Cuts) (width 0.05))
 (segment (start 79.784402 137.0575) (end 79.4815 137.0575) (width 0.381) (layer B.Cu) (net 1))
 (segment (start 81.484402 135.3575) (end 79.784402 137.0575) (width 0.381) (layer B.Cu) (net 1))
 (segment (start 81.6815 135.3575) (end 81.484402 135.3575) (width 0.381) (layer B.Cu) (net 1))
 (segment (start 76.351 137.0575) (end 76.2635 137.145) (width 0.381) (layer B.Cu) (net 1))
 (segment (start 79.4815 137.0575) (end 76.351 137.0575) (width 0.381) (layer B.Cu) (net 1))
 (segment (start 85.447 135.3575) (end 85.5345 135.27) (width 0.381) (layer B.Cu) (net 1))
 (segment (start 81.6815 135.3575) (end 85.447 135.3575) (width 0.381) (layer B.Cu) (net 1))
 (segment (start 88.1045 132.7) (end 88.9 132.7) (width 0.381) (layer B.Cu) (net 1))
 (segment (start 85.5345 135.27) (end 88.1045 132.7) (width 0.381) (layer B.Cu) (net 1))
 (segment (start 89.456237 127.699987) (end 88.9 127.14375) (width 0.381) (layer B.Cu) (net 1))
 (segment (start 90.4875 128.73125) (end 89.456237 127.699987) (width 0.381) (layer B.Cu) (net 1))
 (segment (start 90.4875 131.1125) (end 90.4875 128.73125) (width 0.381) (layer B.Cu) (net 1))
 (segment (start 88.9 132.7) (end 90.4875 131.1125) (width 0.381) (layer B.Cu) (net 1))
 (segment (start 90.4875 121.44375) (end 88.9 119.85625) (width 0.381) (layer B.Cu) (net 1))
 (segment (start 88.9 127.14375) (end 90.4875 125.55625) (width 0.381) (layer B.Cu) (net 1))
 (segment (start 90.4875 125.55625) (end 90.4875 121.44375) (width 0.381) (layer B.Cu) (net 1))
 (segment (start 86.0155 120.2945) (end 84.8845 120.2945) (width 0.381) (layer B.Cu) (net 1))
 (segment (start 87.899 120.2945) (end 86.0155 120.2945) (width 0.381) (layer B.Cu) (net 1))
 (segment (start 88.1 120.0935) (end 87.899 120.2945) (width 0.381) (layer B.Cu) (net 1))
 (segment (start 88.9 120.0935) (end 88.1 120.0935) (width 0.381) (layer B.Cu) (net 1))
 (segment (start 80.7845 125.6635) (end 80.7845 126.7945) (width 0.381) (layer B.Cu) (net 1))
 (segment (start 80.7845 123.2635) (end 80.7845 125.6635) (width 0.381) (layer B.Cu) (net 1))
 (segment (start 83.7535 120.2945) (end 80.7845 123.2635) (width 0.381) (layer B.Cu) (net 1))
 (segment (start 84.8845 120.2945) (end 83.7535 120.2945) (width 0.381) (layer B.Cu) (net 1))
 (segment (start 74.6155 125.0945) (end 73.4845 125.0945) (width 0.381) (layer B.Cu) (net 1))
 (segment (start 76.67875 123.03125) (end 74.6155 125.0945) (width 0.381) (layer B.Cu) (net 1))
 (segment (start 80.7845 123.2635) (end 80.55225 123.03125) (width 0.381) (layer B.Cu) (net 1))
 (segment (start 69.61325 125.0945) (end 69.1515 125.55625) (width 0.381) (layer B.Cu) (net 1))
 (segment (start 73.4845 125.0945) (end 69.61325 125.0945) (width 0.381) (layer B.Cu) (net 1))
 (segment (start 75.9845 122.022) (end 76.99375 123.03125) (width 0.381) (layer B.Cu) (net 1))
 (segment (start 75.9845 115.3945) (end 75.9845 122.022) (width 0.381) (layer B.Cu) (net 1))
 (segment (start 80.55225 123.03125) (end 76.99375 123.03125) (width 0.381) (layer B.Cu) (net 1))
 (segment (start 76.99375 123.03125) (end 76.67875 123.03125) (width 0.381) (layer B.Cu) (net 1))
 (segment (start 80.23125 111.125) (end 80.81875 111.125) (width 0.381) (layer B.Cu) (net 1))
 (segment (start 73.21875 111.125) (end 80.23125 111.125) (width 0.381) (layer B.Cu) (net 1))
 (segment (start 71.45 109.35625) (end 73.21875 111.125) (width 0.381) (layer B.Cu) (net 1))
 (segment (start 71.45 108.48125) (end 71.45 109.35625) (width 0.381) (layer B.Cu) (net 1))
 (segment (start 86.23125 110.325) (end 86.23125 111.125) (width 0.381) (layer B.Cu) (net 1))
 (segment (start 83.859499 107.953249) (end 86.23125 110.325) (width 0.381) (layer B.Cu) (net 1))
 (segment (start 82.964309 107.953249) (end 83.859499 107.953249) (width 0.381) (layer B.Cu) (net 1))
 (segment (start 80.81875 110.098808) (end 82.964309 107.953249) (width 0.381) (layer B.Cu) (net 1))
 (segment (start 80.81875 111.125) (end 80.81875 110.098808) (width 0.381) (layer B.Cu) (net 1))
 (segment (start 89.456237 119.537263) (end 88.9 120.0935) (width 0.381) (layer B.Cu) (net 1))
 (segment (start 89.456237 110.878007) (end 89.456237 119.537263) (width 0.381) (layer B.Cu) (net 1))
 (segment (start 88.61272 110.03449) (end 89.456237 110.878007) (width 0.381) (layer B.Cu) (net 1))
 (segment (start 87.32176 110.03449) (end 88.61272 110.03449) (width 0.381) (layer B.Cu) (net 1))
 (segment (start 86.23125 111.125) (end 87.32176 110.03449) (width 0.381) (layer B.Cu) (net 1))
 (segment (start 76.0765 137.145) (end 76.2635 137.145) (width 0.381) (layer B.Cu) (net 1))
 (segment (start 71.3625 132.431) (end 76.0765 137.145) (width 0.381) (layer B.Cu) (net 1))
 (segment (start 71.3625 131.5) (end 71.3625 132.431) (width 0.381) (layer B.Cu) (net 1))
 (segment (start 79.394 135.27) (end 79.4815 135.3575) (width 0.254) (layer B.Cu) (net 2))
 (segment (start 76.2635 135.27) (end 79.394 135.27) (width 0.254) (layer B.Cu) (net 2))
 (segment (start 81.769 137.145) (end 81.6815 137.0575) (width 0.254) (layer B.Cu) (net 3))
 (segment (start 85.5345 137.145) (end 81.769 137.145) (width 0.254) (layer B.Cu) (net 3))
 (via (at 80.9625 138.90625) (size 0.8) (drill 0.4) (layers F.Cu B.Cu) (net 3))
 (segment (start 81.6815 137.0575) (end 81.6815 138.18725) (width 0.254) (layer B.Cu) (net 3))
 (segment (start 81.6815 138.18725) (end 80.9625 138.90625) (width 0.254) (layer B.Cu) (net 3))
 (via (at 79.375 123.825) (size 0.8) (drill 0.4) (layers F.Cu B.Cu) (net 3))
 (segment (start 80.9625 138.90625) (end 79.375 137.31875) (width 0.254) (layer F.Cu) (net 3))
 (segment (start 79.375 137.31875) (end 79.375 123.825) (width 0.254) (layer F.Cu) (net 3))
 (segment (start 79.9845 124.4345) (end 79.9845 126.7945) (width 0.254) (layer B.Cu) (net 3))
 (segment (start 79.375 123.825) (end 79.9845 124.4345) (width 0.254) (layer B.Cu) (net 3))
 (segment (start 66.675 121.25625) (end 66.675 122.2375) (width 0.381) (layer B.Cu) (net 4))
 (segment (start 66.675 122.2375) (end 68.2625 123.825) (width 0.381) (layer B.Cu) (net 4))
 (segment (start 68.2625 123.825) (end 69.05625 123.825) (width 0.381) (layer B.Cu) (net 4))
 (segment (start 69.52575 124.2945) (end 73.4845 124.2945) (width 0.381) (layer B.Cu) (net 4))
 (segment (start 69.05625 123.825) (end 69.52575 124.2945) (width 0.381) (layer B.Cu) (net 4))
 (via (at 83.34375 108.74375) (size 0.8) (drill 0.4) (layers F.Cu B.Cu) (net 4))
 (segment (start 82.69375 111.125) (end 82.69375 109.39375) (width 0.381) (layer B.Cu) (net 4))
 (segment (start 82.69375 109.39375) (end 83.34375 108.74375) (width 0.381) (layer B.Cu) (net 4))
 (segment (start 81.5845 127.9255) (end 81.5845 126.7945) (width 0.381) (layer B.Cu) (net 4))
 (segment (start 84.118263 130.459263) (end 81.5845 127.9255) (width 0.381) (layer B.Cu) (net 4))
 (segment (start 85.041763 130.459263) (end 84.118263 130.459263) (width 0.381) (layer B.Cu) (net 4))
 (segment (start 85.598 131.0155) (end 85.041763 130.459263) (width 0.381) (layer B.Cu) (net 4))
 (segment (start 85.598 128.57075) (end 88.9 125.26875) (width 0.381) (layer B.Cu) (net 4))
 (segment (start 85.598 131.0155) (end 85.598 128.57075) (width 0.381) (layer B.Cu) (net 4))
 (segment (start 88.9 125.26875) (end 88.9 121.9685) (width 0.381) (layer B.Cu) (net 4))
 (segment (start 88.826 121.8945) (end 88.9 121.9685) (width 0.381) (layer B.Cu) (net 4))
 (segment (start 84.8845 121.8945) (end 88.826 121.8945) (width 0.381) (layer B.Cu) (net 4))
 (via (at 67.46875 110.33125) (size 0.8) (drill 0.4) (layers F.Cu B.Cu) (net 12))
 (segment (start 68.25 108.48125) (end 68.25 109.55) (width 0.381) (layer B.Cu) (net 12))
 (segment (start 68.25 109.55) (end 67.46875 110.33125) (width 0.381) (layer B.Cu) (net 12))
 (segment (start 67.46875 110.33125) (end 65.0875 112.7125) (width 0.381) (layer F.Cu) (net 12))
 (via (at 65.0875 118.26875) (size 0.8) (drill 0.4) (layers F.Cu B.Cu) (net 12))
 (segment (start 65.0875 112.7125) (end 65.0875 118.26875) (width 0.381) (layer F.Cu) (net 12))
 (segment (start 66.4875 118.26875) (end 66.675 118.45625) (width 0.381) (layer B.Cu) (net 12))
 (segment (start 65.0875 118.26875) (end 66.4875 118.26875) (width 0.381) (layer B.Cu) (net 12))
 (via (at 84.93125 112.7125) (size 0.8) (drill 0.4) (layers F.Cu B.Cu) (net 23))
 (segment (start 84.59151 113.05224) (end 84.93125 112.7125) (width 0.254) (layer B.Cu) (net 23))
 (segment (start 66.675 114.15625) (end 67.77901 113.05224) (width 0.254) (layer B.Cu) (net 23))
 (segment (start 67.77901 113.05224) (end 84.59151 113.05224) (width 0.254) (layer B.Cu) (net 23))
 (via (at 84.93125 115.09375) (size 0.8) (drill 0.4) (layers F.Cu B.Cu) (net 23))
 (segment (start 84.93125 112.7125) (end 84.93125 115.09375) (width 0.254) (layer F.Cu) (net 23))
 (segment (start 83.8805 118.6945) (end 84.8845 118.6945) (width 0.254) (layer B.Cu) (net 23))
 (segment (start 83.807499 118.621499) (end 83.8805 118.6945) (width 0.254) (layer B.Cu) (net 23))
 (segment (start 84.93125 115.09375) (end 83.807499 116.217501) (width 0.254) (layer B.Cu) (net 23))
 (segment (start 83.807499 116.217501) (end 83.807499 118.621499) (width 0.254) (layer B.Cu) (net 23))
 (via (at 68.849997 110.33125) (size 0.8) (drill 0.4) (layers F.Cu B.Cu) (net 24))
 (segment (start 69.05 108.48125) (end 69.05 110.131247) (width 0.254) (layer B.Cu) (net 24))
 (segment (start 69.05 110.131247) (end 68.849997 110.33125) (width 0.254) (layer B.Cu) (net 24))
 (segment (start 68.849997 110.33125) (end 68.2625 110.918747) (width 0.254) (layer F.Cu) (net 24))
 (segment (start 68.2625 110.918747) (end 68.2625 116.68125) (width 0.254) (layer F.Cu) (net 24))
 (via (at 68.2625 116.68125) (size 0.8) (drill 0.4) (layers F.Cu B.Cu) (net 24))
 (segment (start 67.6125 116.03125) (end 68.2625 116.68125) (width 0.254) (layer B.Cu) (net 24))
 (segment (start 66.675 116.03125) (end 67.6125 116.03125) (width 0.254) (layer B.Cu) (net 24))
 (via (at 69.85 117.475) (size 0.8) (drill 0.4) (layers F.Cu B.Cu) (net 25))
 (via (at 69.85 110.33125) (size 0.8) (drill 0.4) (layers F.Cu B.Cu) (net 25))
 (segment (start 69.85 111.125) (end 69.05625 111.91875) (width 0.254) (layer F.Cu) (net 25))
 (segment (start 69.05625 111.91875) (end 69.05625 116.68125) (width 0.254) (layer F.Cu) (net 25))
 (segment (start 69.85 117.475) (end 69.85 116.03125) (width 0.254) (layer B.Cu) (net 25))
 (segment (start 69.05625 116.68125) (end 69.85 117.475) (width 0.254) (layer F.Cu) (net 25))
 (segment (start 69.85 110.33125) (end 69.85 111.125) (width 0.254) (layer F.Cu) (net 25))
 (segment (start 69.85 108.48125) (end 69.85 110.33125) (width 0.254) (layer B.Cu) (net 25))
 (segment (start 69.85 114.15625) (end 69.85 113.50625) (width 0.254) (layer B.Cu) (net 26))
 (segment (start 69.85 113.50625) (end 70.64375 114.3) (width 0.254) (layer B.Cu) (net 26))
 (segment (start 70.64375 114.3) (end 85.725 114.3) (width 0.254) (layer B.Cu) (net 26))
 (segment (start 85.8885 119.4945) (end 84.8845 119.4945) (width 0.254) (layer B.Cu) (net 26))
 (segment (start 85.725 114.3) (end 85.961501 114.536501) (width 0.254) (layer B.Cu) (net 26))
 (segment (start 85.961501 114.536501) (end 85.961501 119.421499) (width 0.254) (layer B.Cu) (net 26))
 (segment (start 85.961501 119.421499) (end 85.8885 119.4945) (width 0.254) (layer B.Cu) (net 26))
 (segment (start 84.60725 133.88125) (end 85.598 132.8905) (width 0.254) (layer B.Cu) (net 27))
 (via (at 81.75625 123.825) (size 0.8) (drill 0.4) (layers F.Cu B.Cu) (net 27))
 (segment (start 81.75625 130.175) (end 81.75625 123.825) (width 0.254) (layer F.Cu) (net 27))
 (segment (start 82.3845 124.45325) (end 82.3845 126.7945) (width 0.254) (layer B.Cu) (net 27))
 (segment (start 81.75625 123.825) (end 82.3845 124.45325) (width 0.254) (layer B.Cu) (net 27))
 (via (at 81.75625 132.55625) (size 0.8) (drill 0.4) (layers F.Cu B.Cu) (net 27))
 (segment (start 85.598 132.8905) (end 82.0905 132.8905) (width 0.254) (layer B.Cu) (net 27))
 (segment (start 82.0905 132.8905) (end 81.75625 132.55625) (width 0.254) (layer B.Cu) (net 27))
 (segment (start 81.75625 132.55625) (end 81.75625 130.175) (width 0.254) (layer F.Cu) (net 27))
 (segment (start 81.356251 132.156251) (end 81.75625 132.55625) (width 0.254) (layer B.Cu) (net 27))
 (segment (start 79.822999 130.622999) (end 81.356251 132.156251) (width 0.254) (layer B.Cu) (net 27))
 (segment (start 70.089501 130.622999) (end 79.822999 130.622999) (width 0.254) (layer B.Cu) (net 27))
 (segment (start 65.5125 135.2) (end 70.089501 130.622999) (width 0.254) (layer B.Cu) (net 27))
 (segment (start 65.1625 135.2) (end 65.5125 135.2) (width 0.254) (layer B.Cu) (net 27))
 (via (at 71.4375 118.26875) (size 0.8) (drill 0.4) (layers F.Cu B.Cu) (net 28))
 (segment (start 72.61175 117.0945) (end 73.4845 117.0945) (width 0.254) (layer B.Cu) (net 28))
 (segment (start 71.4375 118.26875) (end 72.61175 117.0945) (width 0.254) (layer B.Cu) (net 28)))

